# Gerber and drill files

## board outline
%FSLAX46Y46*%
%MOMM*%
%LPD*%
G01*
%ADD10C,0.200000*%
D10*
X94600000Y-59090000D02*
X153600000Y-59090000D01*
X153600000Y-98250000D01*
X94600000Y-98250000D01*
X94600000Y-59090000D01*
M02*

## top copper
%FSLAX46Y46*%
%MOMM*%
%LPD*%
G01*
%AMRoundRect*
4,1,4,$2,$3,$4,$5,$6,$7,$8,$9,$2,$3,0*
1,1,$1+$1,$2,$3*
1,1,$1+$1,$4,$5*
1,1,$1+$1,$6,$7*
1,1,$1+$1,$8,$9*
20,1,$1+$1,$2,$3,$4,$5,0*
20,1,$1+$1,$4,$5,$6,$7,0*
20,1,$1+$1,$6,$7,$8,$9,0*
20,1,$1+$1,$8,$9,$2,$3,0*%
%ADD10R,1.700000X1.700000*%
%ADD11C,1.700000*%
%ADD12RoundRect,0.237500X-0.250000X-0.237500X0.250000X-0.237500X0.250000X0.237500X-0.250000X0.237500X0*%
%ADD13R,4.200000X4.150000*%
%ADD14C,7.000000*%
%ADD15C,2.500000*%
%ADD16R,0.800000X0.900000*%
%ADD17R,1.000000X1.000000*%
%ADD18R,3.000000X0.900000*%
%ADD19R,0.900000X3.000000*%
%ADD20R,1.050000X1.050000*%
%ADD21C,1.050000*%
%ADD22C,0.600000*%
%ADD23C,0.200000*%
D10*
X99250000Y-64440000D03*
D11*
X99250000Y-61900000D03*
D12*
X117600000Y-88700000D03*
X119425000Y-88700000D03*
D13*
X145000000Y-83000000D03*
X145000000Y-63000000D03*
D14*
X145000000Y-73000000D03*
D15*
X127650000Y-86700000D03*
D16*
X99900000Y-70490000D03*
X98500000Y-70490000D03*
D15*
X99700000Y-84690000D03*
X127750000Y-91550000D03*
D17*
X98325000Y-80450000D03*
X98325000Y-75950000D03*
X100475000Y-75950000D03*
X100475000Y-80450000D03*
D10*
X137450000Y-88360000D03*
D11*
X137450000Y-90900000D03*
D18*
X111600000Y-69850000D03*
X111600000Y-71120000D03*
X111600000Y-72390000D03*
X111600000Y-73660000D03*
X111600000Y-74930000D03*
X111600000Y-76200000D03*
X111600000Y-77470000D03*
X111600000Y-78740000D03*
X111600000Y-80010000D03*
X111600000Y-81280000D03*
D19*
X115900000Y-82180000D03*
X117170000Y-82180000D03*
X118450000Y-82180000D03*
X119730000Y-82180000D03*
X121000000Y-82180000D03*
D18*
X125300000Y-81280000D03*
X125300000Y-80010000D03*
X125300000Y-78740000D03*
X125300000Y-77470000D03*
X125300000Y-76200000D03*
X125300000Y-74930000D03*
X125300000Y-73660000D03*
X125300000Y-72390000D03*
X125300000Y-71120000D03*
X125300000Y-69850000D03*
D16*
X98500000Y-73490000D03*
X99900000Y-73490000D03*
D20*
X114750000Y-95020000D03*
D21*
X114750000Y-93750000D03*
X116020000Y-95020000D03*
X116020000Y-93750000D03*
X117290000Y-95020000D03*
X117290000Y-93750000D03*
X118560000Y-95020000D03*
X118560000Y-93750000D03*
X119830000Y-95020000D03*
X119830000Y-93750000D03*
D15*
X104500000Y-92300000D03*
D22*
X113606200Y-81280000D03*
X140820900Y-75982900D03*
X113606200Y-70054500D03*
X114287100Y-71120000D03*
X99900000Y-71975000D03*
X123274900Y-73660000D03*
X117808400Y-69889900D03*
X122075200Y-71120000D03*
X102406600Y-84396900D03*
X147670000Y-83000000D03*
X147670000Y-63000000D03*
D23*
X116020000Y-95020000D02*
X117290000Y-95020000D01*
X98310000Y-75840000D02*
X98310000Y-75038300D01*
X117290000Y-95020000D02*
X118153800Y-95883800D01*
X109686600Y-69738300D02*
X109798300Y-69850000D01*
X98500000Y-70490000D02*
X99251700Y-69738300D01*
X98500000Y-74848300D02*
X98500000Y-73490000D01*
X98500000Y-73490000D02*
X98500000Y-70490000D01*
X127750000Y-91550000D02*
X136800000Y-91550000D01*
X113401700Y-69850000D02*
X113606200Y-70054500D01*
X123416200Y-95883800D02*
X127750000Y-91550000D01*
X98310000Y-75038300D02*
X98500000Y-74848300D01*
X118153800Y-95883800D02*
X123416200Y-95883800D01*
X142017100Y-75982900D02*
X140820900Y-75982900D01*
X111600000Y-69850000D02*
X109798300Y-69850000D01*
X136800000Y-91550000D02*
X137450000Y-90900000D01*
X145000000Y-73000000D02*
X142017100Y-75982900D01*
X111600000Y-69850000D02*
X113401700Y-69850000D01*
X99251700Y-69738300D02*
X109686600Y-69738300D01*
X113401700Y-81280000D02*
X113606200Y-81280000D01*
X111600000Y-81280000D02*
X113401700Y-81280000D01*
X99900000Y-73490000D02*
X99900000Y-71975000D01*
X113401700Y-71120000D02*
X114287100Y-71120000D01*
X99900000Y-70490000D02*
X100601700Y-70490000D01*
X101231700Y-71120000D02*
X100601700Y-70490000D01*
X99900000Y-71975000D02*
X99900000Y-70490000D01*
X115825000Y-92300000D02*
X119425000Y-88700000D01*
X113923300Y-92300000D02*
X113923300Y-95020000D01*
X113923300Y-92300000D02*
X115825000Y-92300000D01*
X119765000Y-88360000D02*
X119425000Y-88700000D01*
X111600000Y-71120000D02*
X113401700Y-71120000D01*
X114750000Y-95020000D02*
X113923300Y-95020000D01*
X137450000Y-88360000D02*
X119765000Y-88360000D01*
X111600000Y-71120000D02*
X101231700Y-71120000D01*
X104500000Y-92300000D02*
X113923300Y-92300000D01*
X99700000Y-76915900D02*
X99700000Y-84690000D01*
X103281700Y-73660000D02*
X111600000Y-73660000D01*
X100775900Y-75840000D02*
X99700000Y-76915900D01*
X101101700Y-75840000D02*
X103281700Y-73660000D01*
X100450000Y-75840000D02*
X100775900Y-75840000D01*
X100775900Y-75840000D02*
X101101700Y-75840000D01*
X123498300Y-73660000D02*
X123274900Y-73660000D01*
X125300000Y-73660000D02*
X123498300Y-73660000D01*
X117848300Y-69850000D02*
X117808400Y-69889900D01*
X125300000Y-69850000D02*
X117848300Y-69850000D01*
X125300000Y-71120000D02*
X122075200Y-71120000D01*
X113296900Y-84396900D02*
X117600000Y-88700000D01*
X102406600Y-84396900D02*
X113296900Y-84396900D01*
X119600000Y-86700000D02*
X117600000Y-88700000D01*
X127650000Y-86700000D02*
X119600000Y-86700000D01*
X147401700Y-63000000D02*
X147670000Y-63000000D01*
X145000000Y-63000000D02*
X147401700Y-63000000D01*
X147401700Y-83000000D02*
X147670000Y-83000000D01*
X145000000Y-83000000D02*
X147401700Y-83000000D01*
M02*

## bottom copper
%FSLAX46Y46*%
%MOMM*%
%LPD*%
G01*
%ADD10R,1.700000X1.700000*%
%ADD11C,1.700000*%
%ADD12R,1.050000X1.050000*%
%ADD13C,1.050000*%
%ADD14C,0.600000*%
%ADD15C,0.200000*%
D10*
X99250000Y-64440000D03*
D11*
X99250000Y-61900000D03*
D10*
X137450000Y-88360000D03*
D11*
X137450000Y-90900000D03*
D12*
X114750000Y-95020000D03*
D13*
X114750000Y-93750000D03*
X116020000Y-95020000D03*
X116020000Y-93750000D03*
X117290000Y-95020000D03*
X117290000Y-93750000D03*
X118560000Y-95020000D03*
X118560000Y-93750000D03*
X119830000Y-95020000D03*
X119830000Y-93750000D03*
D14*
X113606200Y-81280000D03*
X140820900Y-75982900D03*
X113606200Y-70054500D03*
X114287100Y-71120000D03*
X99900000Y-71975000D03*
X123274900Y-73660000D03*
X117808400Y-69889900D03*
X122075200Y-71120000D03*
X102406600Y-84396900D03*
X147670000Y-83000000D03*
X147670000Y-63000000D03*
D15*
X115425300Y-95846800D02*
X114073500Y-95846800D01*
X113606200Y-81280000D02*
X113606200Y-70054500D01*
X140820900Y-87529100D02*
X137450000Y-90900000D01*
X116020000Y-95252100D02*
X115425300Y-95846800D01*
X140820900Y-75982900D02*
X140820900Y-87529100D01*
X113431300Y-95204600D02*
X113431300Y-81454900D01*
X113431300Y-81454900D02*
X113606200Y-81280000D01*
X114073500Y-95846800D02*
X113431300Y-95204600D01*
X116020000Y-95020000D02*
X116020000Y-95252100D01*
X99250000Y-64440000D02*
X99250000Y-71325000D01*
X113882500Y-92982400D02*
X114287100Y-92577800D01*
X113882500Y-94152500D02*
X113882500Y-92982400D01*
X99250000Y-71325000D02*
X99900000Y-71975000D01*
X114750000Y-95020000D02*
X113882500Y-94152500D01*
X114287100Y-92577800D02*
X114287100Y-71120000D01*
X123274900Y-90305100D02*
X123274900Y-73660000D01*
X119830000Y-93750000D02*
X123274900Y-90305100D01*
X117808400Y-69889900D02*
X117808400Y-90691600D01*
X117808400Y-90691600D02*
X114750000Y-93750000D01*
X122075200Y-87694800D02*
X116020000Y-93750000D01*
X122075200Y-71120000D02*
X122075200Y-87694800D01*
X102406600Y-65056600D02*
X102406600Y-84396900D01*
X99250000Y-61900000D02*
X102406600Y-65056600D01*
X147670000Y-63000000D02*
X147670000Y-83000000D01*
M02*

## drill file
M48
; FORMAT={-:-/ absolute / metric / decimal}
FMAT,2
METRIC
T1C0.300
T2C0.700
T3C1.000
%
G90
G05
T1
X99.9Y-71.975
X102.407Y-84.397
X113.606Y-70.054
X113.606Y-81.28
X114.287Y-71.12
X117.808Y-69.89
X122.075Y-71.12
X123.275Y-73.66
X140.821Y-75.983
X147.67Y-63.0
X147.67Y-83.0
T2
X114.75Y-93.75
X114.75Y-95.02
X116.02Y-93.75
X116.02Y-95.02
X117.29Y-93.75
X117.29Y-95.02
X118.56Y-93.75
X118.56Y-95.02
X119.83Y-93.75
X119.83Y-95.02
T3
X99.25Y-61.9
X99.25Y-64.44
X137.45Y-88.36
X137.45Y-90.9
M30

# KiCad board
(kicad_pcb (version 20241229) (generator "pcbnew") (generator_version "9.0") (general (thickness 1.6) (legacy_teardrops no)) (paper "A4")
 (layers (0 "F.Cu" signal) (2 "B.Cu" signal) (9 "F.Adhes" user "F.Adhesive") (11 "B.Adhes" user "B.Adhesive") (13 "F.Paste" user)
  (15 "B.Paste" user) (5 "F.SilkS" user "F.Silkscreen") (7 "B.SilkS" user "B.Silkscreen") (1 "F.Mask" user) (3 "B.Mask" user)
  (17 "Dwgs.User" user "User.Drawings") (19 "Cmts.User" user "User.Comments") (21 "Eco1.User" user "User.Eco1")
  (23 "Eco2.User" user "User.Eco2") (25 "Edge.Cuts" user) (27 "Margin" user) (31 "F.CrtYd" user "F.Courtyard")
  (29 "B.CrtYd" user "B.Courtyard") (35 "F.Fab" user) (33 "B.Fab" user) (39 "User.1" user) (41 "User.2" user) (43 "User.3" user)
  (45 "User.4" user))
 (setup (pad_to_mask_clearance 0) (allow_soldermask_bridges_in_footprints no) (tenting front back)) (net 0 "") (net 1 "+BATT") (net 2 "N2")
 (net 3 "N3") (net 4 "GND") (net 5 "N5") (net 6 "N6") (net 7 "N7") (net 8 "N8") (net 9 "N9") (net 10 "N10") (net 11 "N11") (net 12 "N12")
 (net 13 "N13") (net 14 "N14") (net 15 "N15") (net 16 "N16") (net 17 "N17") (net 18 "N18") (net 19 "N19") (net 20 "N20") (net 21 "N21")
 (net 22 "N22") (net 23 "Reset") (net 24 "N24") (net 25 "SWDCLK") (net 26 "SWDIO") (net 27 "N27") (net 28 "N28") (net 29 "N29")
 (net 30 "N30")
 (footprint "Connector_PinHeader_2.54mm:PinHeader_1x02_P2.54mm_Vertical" (layer "F.Cu") (at 99.25 64.44 180)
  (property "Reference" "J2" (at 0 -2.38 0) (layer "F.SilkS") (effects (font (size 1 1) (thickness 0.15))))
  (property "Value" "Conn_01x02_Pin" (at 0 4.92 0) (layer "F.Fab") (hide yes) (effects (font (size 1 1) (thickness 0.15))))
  (pad "1" thru_hole rect (at 0 0 180) (size 1.7 1.7) (drill 1) (layers "*.Cu" "*.Mask") (remove_unused_layers no) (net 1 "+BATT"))
  (pad "2" thru_hole circle (at 0 2.54 180) (size 1.7 1.7) (drill 1) (layers "*.Cu" "*.Mask") (remove_unused_layers no) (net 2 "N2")))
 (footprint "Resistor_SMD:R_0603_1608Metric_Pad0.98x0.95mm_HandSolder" (layer "F.Cu") (at 118.5125 88.7)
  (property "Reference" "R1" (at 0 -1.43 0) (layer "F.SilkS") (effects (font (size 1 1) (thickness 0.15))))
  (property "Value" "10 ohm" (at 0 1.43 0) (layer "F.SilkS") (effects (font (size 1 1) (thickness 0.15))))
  (pad "1" smd roundrect (at -0.9125 0) (size 0.975 0.95) (layers "F.Cu" "F.Mask" "F.Paste") (roundrect_rratio 0.25) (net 2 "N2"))
  (pad "2" smd roundrect (at 0.9125 0) (size 0.975 0.95) (layers "F.Cu" "F.Mask" "F.Paste") (roundrect_rratio 0.25) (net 1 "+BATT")))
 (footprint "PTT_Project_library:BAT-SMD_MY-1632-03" (layer "F.Cu") (at 145 73 90)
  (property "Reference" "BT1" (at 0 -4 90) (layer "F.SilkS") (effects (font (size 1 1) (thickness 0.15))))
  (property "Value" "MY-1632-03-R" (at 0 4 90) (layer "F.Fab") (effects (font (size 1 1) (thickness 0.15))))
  (pad "1" smd rect (at -10 0 90) (size 4.15 4.2) (layers "F.Cu" "F.Mask" "F.Paste") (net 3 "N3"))
  (pad "1" smd rect (at 10 0 90) (size 4.15 4.2) (layers "F.Cu" "F.Mask" "F.Paste") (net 3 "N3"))
  (pad "2" smd circle (at 0 0 90) (size 7 7) (layers "F.Cu" "F.Mask" "F.Paste") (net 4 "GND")))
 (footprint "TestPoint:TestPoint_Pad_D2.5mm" (layer "F.Cu") (at 127.65 86.7 180)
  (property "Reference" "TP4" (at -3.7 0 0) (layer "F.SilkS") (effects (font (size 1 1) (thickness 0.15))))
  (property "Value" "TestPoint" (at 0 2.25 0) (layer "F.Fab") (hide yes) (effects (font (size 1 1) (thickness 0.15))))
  (pad "1" smd circle (at 0 0 180) (size 2.5 2.5) (layers "F.Cu" "F.Mask") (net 2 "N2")))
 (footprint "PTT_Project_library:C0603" (layer "F.Cu") (at 99.2 70.49 180)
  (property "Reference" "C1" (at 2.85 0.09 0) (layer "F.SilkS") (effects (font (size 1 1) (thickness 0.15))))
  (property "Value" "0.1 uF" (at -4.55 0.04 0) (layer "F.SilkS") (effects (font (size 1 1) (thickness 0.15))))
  (pad "1" smd rect (at -0.7 0 180) (size 0.8 0.9) (layers "F.Cu" "F.Mask" "F.Paste") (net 1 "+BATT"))
  (pad "2" smd rect (at 0.7 0 180) (size 0.8 0.9) (layers "F.Cu" "F.Mask" "F.Paste") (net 4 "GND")))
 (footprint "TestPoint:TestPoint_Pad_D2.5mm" (layer "F.Cu") (at 99.7 84.69)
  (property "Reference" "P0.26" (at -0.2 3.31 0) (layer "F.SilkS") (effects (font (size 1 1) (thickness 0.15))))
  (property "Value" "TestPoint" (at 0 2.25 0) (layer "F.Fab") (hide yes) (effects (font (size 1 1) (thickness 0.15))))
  (pad "1" smd circle (at 0 0) (size 2.5 2.5) (layers "F.Cu" "F.Mask") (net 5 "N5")))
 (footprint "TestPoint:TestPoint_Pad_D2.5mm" (layer "F.Cu") (at 127.75 91.55)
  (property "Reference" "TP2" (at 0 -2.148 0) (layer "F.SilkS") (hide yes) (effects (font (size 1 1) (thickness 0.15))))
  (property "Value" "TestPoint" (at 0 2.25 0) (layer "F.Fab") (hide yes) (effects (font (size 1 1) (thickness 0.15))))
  (pad "1" smd circle (at 0 0) (size 2.5 2.5) (layers "F.Cu" "F.Mask") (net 4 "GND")))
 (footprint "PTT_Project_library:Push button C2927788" (layer "F.Cu") (at 99.4 78.2 90)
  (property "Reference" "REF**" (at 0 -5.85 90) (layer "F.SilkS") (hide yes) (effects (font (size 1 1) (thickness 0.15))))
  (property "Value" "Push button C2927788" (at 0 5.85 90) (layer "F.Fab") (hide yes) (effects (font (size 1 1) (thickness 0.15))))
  (pad "1" smd rect (at -2.25 -1.075 90) (size 1 1) (layers "F.Cu" "F.Mask" "F.Paste"))
  (pad "2" smd rect (at 2.25 -1.075 90) (size 1 1) (layers "F.Cu" "F.Mask" "F.Paste"))
  (pad "3" smd rect (at 2.25 1.075 90) (size 1 1) (layers "F.Cu" "F.Mask" "F.Paste"))
  (pad "4" smd rect (at -2.25 1.075 90) (size 1 1) (layers "F.Cu" "F.Mask" "F.Paste")))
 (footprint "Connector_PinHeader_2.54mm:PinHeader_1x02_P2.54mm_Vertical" (layer "F.Cu") (at 137.45 88.36)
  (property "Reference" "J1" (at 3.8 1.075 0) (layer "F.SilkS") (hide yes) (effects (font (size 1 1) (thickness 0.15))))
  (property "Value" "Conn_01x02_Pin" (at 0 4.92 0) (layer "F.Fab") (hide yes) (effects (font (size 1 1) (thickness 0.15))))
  (pad "1" thru_hole rect (at 0 0) (size 1.7 1.7) (drill 1) (layers "*.Cu" "*.Mask") (remove_unused_layers no) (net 1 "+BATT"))
  (pad "2" thru_hole circle (at 0 2.54) (size 1.7 1.7) (drill 1) (layers "*.Cu" "*.Mask") (remove_unused_layers no) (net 4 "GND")))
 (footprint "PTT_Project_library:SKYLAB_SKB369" (layer "F.Cu") (at 118.45 73.48)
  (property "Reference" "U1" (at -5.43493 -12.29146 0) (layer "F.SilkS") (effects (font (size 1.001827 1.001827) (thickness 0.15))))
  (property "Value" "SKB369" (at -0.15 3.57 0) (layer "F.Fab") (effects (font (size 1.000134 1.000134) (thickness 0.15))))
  (pad "1" smd rect (at -6.85 -3.63) (size 3 0.9) (layers "F.Cu" "F.Mask" "F.Paste") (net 4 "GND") (solder_mask_margin 0.102))
  (pad "2" smd rect (at -6.85 -2.36) (size 3 0.9) (layers "F.Cu" "F.Mask" "F.Paste") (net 1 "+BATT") (solder_mask_margin 0.102))
  (pad "3" smd rect (at -6.85 -1.09) (size 3 0.9) (layers "F.Cu" "F.Mask" "F.Paste") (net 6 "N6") (solder_mask_margin 0.102))
  (pad "4" smd rect (at -6.85 0.18) (size 3 0.9) (layers "F.Cu" "F.Mask" "F.Paste") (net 5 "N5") (solder_mask_margin 0.102))
  (pad "5" smd rect (at -6.85 1.45) (size 3 0.9) (layers "F.Cu" "F.Mask" "F.Paste") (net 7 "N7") (solder_mask_margin 0.102))
  (pad "6" smd rect (at -6.85 2.72) (size 3 0.9) (layers "F.Cu" "F.Mask" "F.Paste") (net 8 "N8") (solder_mask_margin 0.102))
  (pad "7" smd rect (at -6.85 3.99) (size 3 0.9) (layers "F.Cu" "F.Mask" "F.Paste") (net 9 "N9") (solder_mask_margin 0.102))
  (pad "8" smd rect (at -6.85 5.26) (size 3 0.9) (layers "F.Cu" "F.Mask" "F.Paste") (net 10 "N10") (solder_mask_margin 0.102))
  (pad "9" smd rect (at -6.85 6.53) (size 3 0.9) (layers "F.Cu" "F.Mask" "F.Paste") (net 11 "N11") (solder_mask_margin 0.102))
  (pad "10" smd rect (at -6.85 7.8) (size 3 0.9) (layers "F.Cu" "F.Mask" "F.Paste") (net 4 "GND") (solder_mask_margin 0.102))
  (pad "11" smd rect (at -2.55 8.7) (size 0.9 3) (layers "F.Cu" "F.Mask" "F.Paste") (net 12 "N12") (solder_mask_margin 0.102))
  (pad "12" smd rect (at -1.28 8.7) (size 0.9 3) (layers "F.Cu" "F.Mask" "F.Paste") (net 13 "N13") (solder_mask_margin 0.102))
  (pad "13" smd rect (at 0 8.7) (size 0.9 3) (layers "F.Cu" "F.Mask" "F.Paste") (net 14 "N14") (solder_mask_margin 0.102))
  (pad "14" smd rect (at 1.28 8.7) (size 0.9 3) (layers "F.Cu" "F.Mask" "F.Paste") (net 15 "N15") (solder_mask_margin 0.102))
  (pad "15" smd rect (at 2.55 8.7) (size 0.9 3) (layers "F.Cu" "F.Mask" "F.Paste") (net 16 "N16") (solder_mask_margin 0.102))
  (pad "16" smd rect (at 6.85 7.8) (size 3 0.9) (layers "F.Cu" "F.Mask" "F.Paste") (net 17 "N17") (solder_mask_margin 0.102))
  (pad "17" smd rect (at 6.85 6.53) (size 3 0.9) (layers "F.Cu" "F.Mask" "F.Paste") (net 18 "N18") (solder_mask_margin 0.102))
  (pad "18" smd rect (at 6.85 5.26) (size 3 0.9) (layers "F.Cu" "F.Mask" "F.Paste") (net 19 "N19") (solder_mask_margin 0.102))
  (pad "19" smd rect (at 6.85 3.99) (size 3 0.9) (layers "F.Cu" "F.Mask" "F.Paste") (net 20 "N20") (solder_mask_margin 0.102))
  (pad "20" smd rect (at 6.85 2.72) (size 3 0.9) (layers "F.Cu" "F.Mask" "F.Paste") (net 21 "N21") (solder_mask_margin 0.102))
  (pad "21" smd rect (at 6.85 1.45) (size 3 0.9) (layers "F.Cu" "F.Mask" "F.Paste") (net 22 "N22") (solder_mask_margin 0.102))
  (pad "22" smd rect (at 6.85 0.18) (size 3 0.9) (layers "F.Cu" "F.Mask" "F.Paste") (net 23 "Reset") (solder_mask_margin 0.102))
  (pad "23" smd rect (at 6.85 -1.09) (size 3 0.9) (layers "F.Cu" "F.Mask" "F.Paste") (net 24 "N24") (solder_mask_margin 0.102))
  (pad "24" smd rect (at 6.85 -2.36) (size 3 0.9) (layers "F.Cu" "F.Mask" "F.Paste") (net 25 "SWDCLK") (solder_mask_margin 0.102))
  (pad "25" smd rect (at 6.85 -3.63) (size 3 0.9) (layers "F.Cu" "F.Mask" "F.Paste") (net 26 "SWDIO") (solder_mask_margin 0.102))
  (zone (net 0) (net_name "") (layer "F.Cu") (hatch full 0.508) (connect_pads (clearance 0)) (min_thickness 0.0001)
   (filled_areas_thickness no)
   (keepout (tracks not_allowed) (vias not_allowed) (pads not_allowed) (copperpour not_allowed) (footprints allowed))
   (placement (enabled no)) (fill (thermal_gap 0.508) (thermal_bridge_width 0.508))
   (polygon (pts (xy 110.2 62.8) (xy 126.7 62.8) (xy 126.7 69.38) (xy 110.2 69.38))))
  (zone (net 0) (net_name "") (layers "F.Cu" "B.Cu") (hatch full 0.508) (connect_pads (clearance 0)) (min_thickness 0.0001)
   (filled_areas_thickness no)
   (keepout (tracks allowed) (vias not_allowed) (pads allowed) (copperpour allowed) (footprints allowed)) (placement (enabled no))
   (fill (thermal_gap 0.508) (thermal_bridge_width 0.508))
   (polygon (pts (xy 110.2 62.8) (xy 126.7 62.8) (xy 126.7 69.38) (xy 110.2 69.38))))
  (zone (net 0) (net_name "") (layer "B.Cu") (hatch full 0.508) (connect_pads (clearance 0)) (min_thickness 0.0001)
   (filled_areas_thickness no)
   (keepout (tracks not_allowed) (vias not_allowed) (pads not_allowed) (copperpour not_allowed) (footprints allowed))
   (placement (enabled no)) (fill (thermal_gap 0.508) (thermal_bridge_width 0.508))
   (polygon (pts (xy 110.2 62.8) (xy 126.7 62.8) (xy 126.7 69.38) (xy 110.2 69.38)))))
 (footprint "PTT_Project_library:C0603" (layer "F.Cu") (at 99.2 73.49)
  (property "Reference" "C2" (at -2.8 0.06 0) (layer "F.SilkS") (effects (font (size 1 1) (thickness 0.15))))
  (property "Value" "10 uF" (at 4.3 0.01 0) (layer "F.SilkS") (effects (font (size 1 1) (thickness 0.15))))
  (pad "1" smd rect (at -0.7 0) (size 0.8 0.9) (layers "F.Cu" "F.Mask" "F.Paste") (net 4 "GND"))
  (pad "2" smd rect (at 0.7 0) (size 0.8 0.9) (layers "F.Cu" "F.Mask" "F.Paste") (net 1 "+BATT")))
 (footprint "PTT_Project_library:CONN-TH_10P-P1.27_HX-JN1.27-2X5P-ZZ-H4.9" (layer "F.Cu") (at 117.29 94.39)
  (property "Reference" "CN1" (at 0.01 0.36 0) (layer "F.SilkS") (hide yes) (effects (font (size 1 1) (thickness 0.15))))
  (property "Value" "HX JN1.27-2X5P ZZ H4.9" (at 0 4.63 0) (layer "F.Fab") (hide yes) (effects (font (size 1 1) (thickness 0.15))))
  (pad "1" thru_hole rect (at -2.54 0.63) (size 1.05 1.05) (drill 0.700024) (layers "*.Cu" "*.Mask") (remove_unused_layers no)
   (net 1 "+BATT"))
  (pad "2" thru_hole circle (at -2.54 -0.64) (size 1.05 1.05) (drill 0.700024) (layers "*.Cu" "*.Mask") (remove_unused_layers no)
   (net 26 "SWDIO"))
  (pad "3" thru_hole circle (at -1.27 0.63) (size 1.05 1.05) (drill 0.700024) (layers "*.Cu" "*.Mask") (remove_unused_layers no)
   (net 4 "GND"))
  (pad "4" thru_hole circle (at -1.27 -0.64) (size 1.05 1.05) (drill 0.700024) (layers "*.Cu" "*.Mask") (remove_unused_layers no)
   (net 25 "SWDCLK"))
  (pad "5" thru_hole circle (at 0 0.63) (size 1.05 1.05) (drill 0.700024) (layers "*.Cu" "*.Mask") (remove_unused_layers no) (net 4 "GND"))
  (pad "6" thru_hole circle (at 0 -0.64) (size 1.05 1.05) (drill 0.700024) (layers "*.Cu" "*.Mask") (remove_unused_layers no) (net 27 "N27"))
  (pad "7" thru_hole circle (at 1.27 0.63) (size 1.05 1.05) (drill 0.700024) (layers "*.Cu" "*.Mask") (remove_unused_layers no)
   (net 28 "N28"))
  (pad "8" thru_hole circle (at 1.27 -0.64) (size 1.05 1.05) (drill 0.700024) (layers "*.Cu" "*.Mask") (remove_unused_layers no)
   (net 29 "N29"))
  (pad "9" thru_hole circle (at 2.54 0.63) (size 1.05 1.05) (drill 0.700024) (layers "*.Cu" "*.Mask") (remove_unused_layers no)
   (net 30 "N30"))
  (pad "10" thru_hole circle (at 2.54 -0.64) (size 1.05 1.05) (drill 0.700024) (layers "*.Cu" "*.Mask") (remove_unused_layers no)
   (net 23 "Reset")))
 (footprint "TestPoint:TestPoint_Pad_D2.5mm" (layer "F.Cu") (at 104.5 92.3)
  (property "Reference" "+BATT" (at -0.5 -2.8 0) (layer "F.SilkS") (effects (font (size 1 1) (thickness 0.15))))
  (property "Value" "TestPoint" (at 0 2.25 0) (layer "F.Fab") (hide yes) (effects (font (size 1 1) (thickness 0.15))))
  (pad "1" smd circle (at 0 0) (size 2.5 2.5) (layers "F.Cu" "F.Mask") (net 1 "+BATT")))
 (gr_rect (start 94.6 59.09) (end 153.6 98.25) (stroke (width 0.2) (type solid)) (fill no) (layer "Edge.Cuts"))
 (segment (start 116.02 95.02) (end 117.29 95.02) (width 0.2) (layer "F.Cu") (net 4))
 (segment (start 98.31 75.84) (end 98.31 75.0383) (width 0.2) (layer "F.Cu") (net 4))
 (segment (start 117.29 95.02) (end 118.1538 95.8838) (width 0.2) (layer "F.Cu") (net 4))
 (segment (start 109.6866 69.7383) (end 109.7983 69.85) (width 0.2) (layer "F.Cu") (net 4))
 (segment (start 98.5 70.49) (end 99.2517 69.7383) (width 0.2) (layer "F.Cu") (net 4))
 (segment (start 98.5 74.8483) (end 98.5 73.49) (width 0.2) (layer "F.Cu") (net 4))
 (segment (start 98.5 73.49) (end 98.5 70.49) (width 0.2) (layer "F.Cu") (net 4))
 (segment (start 127.75 91.55) (end 136.8 91.55) (width 0.2) (layer "F.Cu") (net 4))
 (segment (start 113.4017 69.85) (end 113.6062 70.0545) (width 0.2) (layer "F.Cu") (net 4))
 (segment (start 123.4162 95.8838) (end 127.75 91.55) (width 0.2) (layer "F.Cu") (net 4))
 (segment (start 98.31 75.0383) (end 98.5 74.8483) (width 0.2) (layer "F.Cu") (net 4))
 (segment (start 118.1538 95.8838) (end 123.4162 95.8838) (width 0.2) (layer "F.Cu") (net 4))
 (segment (start 142.0171 75.9829) (end 140.8209 75.9829) (width 0.2) (layer "F.Cu") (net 4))
 (segment (start 111.6 69.85) (end 109.7983 69.85) (width 0.2) (layer "F.Cu") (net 4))
 (segment (start 136.8 91.55) (end 137.45 90.9) (width 0.2) (layer "F.Cu") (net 4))
 (segment (start 145 73) (end 142.0171 75.9829) (width 0.2) (layer "F.Cu") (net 4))
 (segment (start 111.6 69.85) (end 113.4017 69.85) (width 0.2) (layer "F.Cu") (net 4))
 (segment (start 99.2517 69.7383) (end 109.6866 69.7383) (width 0.2) (layer "F.Cu") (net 4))
 (segment (start 113.4017 81.28) (end 113.6062 81.28) (width 0.2) (layer "F.Cu") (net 4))
 (segment (start 111.6 81.28) (end 113.4017 81.28) (width 0.2) (layer "F.Cu") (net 4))
 (via (at 113.6062 81.28) (size 0.6) (drill 0.3) (layers "F.Cu" "B.Cu") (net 4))
 (via (at 140.8209 75.9829) (size 0.6) (drill 0.3) (layers "F.Cu" "B.Cu") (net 4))
 (via (at 113.6062 70.0545) (size 0.6) (drill 0.3) (layers "F.Cu" "B.Cu") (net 4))
 (segment (start 115.4253 95.8468) (end 114.0735 95.8468) (width 0.2) (layer "B.Cu") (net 4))
 (segment (start 113.6062 81.28) (end 113.6062 70.0545) (width 0.2) (layer "B.Cu") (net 4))
 (segment (start 140.8209 87.5291) (end 137.45 90.9) (width 0.2) (layer "B.Cu") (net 4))
 (segment (start 116.02 95.2521) (end 115.4253 95.8468) (width 0.2) (layer "B.Cu") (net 4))
 (segment (start 140.8209 75.9829) (end 140.8209 87.5291) (width 0.2) (layer "B.Cu") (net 4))
 (segment (start 113.4313 95.2046) (end 113.4313 81.4549) (width 0.2) (layer "B.Cu") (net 4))
 (segment (start 113.4313 81.4549) (end 113.6062 81.28) (width 0.2) (layer "B.Cu") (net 4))
 (segment (start 114.0735 95.8468) (end 113.4313 95.2046) (width 0.2) (layer "B.Cu") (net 4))
 (segment (start 116.02 95.02) (end 116.02 95.2521) (width 0.2) (layer "B.Cu") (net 4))
 (segment (start 99.9 73.49) (end 99.9 71.975) (width 0.2) (layer "F.Cu") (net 1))
 (segment (start 113.4017 71.12) (end 114.2871 71.12) (width 0.2) (layer "F.Cu") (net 1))
 (segment (start 99.9 70.49) (end 100.6017 70.49) (width 0.2) (layer "F.Cu") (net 1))
 (segment (start 101.2317 71.12) (end 100.6017 70.49) (width 0.2) (layer "F.Cu") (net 1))
 (segment (start 99.9 71.975) (end 99.9 70.49) (width 0.2) (layer "F.Cu") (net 1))
 (segment (start 115.825 92.3) (end 119.425 88.7) (width 0.2) (layer "F.Cu") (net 1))
 (segment (start 113.9233 92.3) (end 113.9233 95.02) (width 0.2) (layer "F.Cu") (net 1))
 (segment (start 113.9233 92.3) (end 115.825 92.3) (width 0.2) (layer "F.Cu") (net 1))
 (segment (start 119.765 88.36) (end 119.425 88.7) (width 0.2) (layer "F.Cu") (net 1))
 (segment (start 111.6 71.12) (end 113.4017 71.12) (width 0.2) (layer "F.Cu") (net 1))
 (segment (start 114.75 95.02) (end 113.9233 95.02) (width 0.2) (layer "F.Cu") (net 1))
 (segment (start 137.45 88.36) (end 119.765 88.36) (width 0.2) (layer "F.Cu") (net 1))
 (segment (start 111.6 71.12) (end 101.2317 71.12) (width 0.2) (layer "F.Cu") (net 1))
 (segment (start 104.5 92.3) (end 113.9233 92.3) (width 0.2) (layer "F.Cu") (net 1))
 (via (at 114.2871 71.12) (size 0.6) (drill 0.3) (layers "F.Cu" "B.Cu") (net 1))
 (via (at 99.9 71.975) (size 0.6) (drill 0.3) (layers "F.Cu" "B.Cu") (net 1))
 (segment (start 99.25 64.44) (end 99.25 71.325) (width 0.2) (layer "B.Cu") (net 1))
 (segment (start 113.8825 92.9824) (end 114.2871 92.5778) (width 0.2) (layer "B.Cu") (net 1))
 (segment (start 113.8825 94.1525) (end 113.8825 92.9824) (width 0.2) (layer "B.Cu") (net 1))
 (segment (start 99.25 71.325) (end 99.9 71.975) (width 0.2) (layer "B.Cu") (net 1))
 (segment (start 114.75 95.02) (end 113.8825 94.1525) (width 0.2) (layer "B.Cu") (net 1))
 (segment (start 114.2871 92.5778) (end 114.2871 71.12) (width 0.2) (layer "B.Cu") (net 1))
 (segment (start 99.7 76.9159) (end 99.7 84.69) (width 0.2) (layer "F.Cu") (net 5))
 (segment (start 103.2817 73.66) (end 111.6 73.66) (width 0.2) (layer "F.Cu") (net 5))
 (segment (start 100.7759 75.84) (end 99.7 76.9159) (width 0.2) (layer "F.Cu") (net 5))
 (segment (start 101.1017 75.84) (end 103.2817 73.66) (width 0.2) (layer "F.Cu") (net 5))
 (segment (start 100.45 75.84) (end 100.7759 75.84) (width 0.2) (layer "F.Cu") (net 5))
 (segment (start 100.7759 75.84) (end 101.1017 75.84) (width 0.2) (layer "F.Cu") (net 5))
 (segment (start 123.4983 73.66) (end 123.2749 73.66) (width 0.2) (layer "F.Cu") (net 23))
 (segment (start 125.3 73.66) (end 123.4983 73.66) (width 0.2) (layer "F.Cu") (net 23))
 (via (at 123.2749 73.66) (size 0.6) (drill 0.3) (layers "F.Cu" "B.Cu") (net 23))
 (segment (start 123.2749 90.3051) (end 123.2749 73.66) (width 0.2) (layer "B.Cu") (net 23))
 (segment (start 119.83 93.75) (end 123.2749 90.3051) (width 0.2) (layer "B.Cu") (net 23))
 (segment (start 117.8483 69.85) (end 117.8084 69.8899) (width 0.2) (layer "F.Cu") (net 26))
 (segment (start 125.3 69.85) (end 117.8483 69.85) (width 0.2) (layer "F.Cu") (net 26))
 (via (at 117.8084 69.8899) (size 0.6) (drill 0.3) (layers "F.Cu" "B.Cu") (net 26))
 (segment (start 117.8084 69.8899) (end 117.8084 90.6916) (width 0.2) (layer "B.Cu") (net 26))
 (segment (start 117.8084 90.6916) (end 114.75 93.75) (width 0.2) (layer "B.Cu") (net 26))
 (segment (start 125.3 71.12) (end 122.0752 71.12) (width 0.2) (layer "F.Cu") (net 25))
 (via (at 122.0752 71.12) (size 0.6) (drill 0.3) (layers "F.Cu" "B.Cu") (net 25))
 (segment (start 122.0752 87.6948) (end 116.02 93.75) (width 0.2) (layer "B.Cu") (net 25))
 (segment (start 122.0752 71.12) (end 122.0752 87.6948) (width 0.2) (layer "B.Cu") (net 25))
 (segment (start 113.2969 84.3969) (end 117.6 88.7) (width 0.2) (layer "F.Cu") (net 2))
 (segment (start 102.4066 84.3969) (end 113.2969 84.3969) (width 0.2) (layer "F.Cu") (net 2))
 (segment (start 119.6 86.7) (end 117.6 88.7) (width 0.2) (layer "F.Cu") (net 2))
 (segment (start 127.65 86.7) (end 119.6 86.7) (width 0.2) (layer "F.Cu") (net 2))
 (via (at 102.4066 84.3969) (size 0.6) (drill 0.3) (layers "F.Cu" "B.Cu") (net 2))
 (segment (start 102.4066 65.0566) (end 102.4066 84.3969) (width 0.2) (layer "B.Cu") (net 2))
 (segment (start 99.25 61.9) (end 102.4066 65.0566) (width 0.2) (layer "B.Cu") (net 2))
 (segment (start 147.4017 63) (end 147.67 63) (width 0.2) (layer "F.Cu") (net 3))
 (segment (start 145 63) (end 147.4017 63) (width 0.2) (layer "F.Cu") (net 3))
 (segment (start 147.4017 83) (end 147.67 83) (width 0.2) (layer "F.Cu") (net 3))
 (segment (start 145 83) (end 147.4017 83) (width 0.2) (layer "F.Cu") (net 3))
 (via (at 147.67 83) (size 0.6) (drill 0.3) (layers "F.Cu" "B.Cu") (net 3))
 (via (at 147.67 63) (size 0.6) (drill 0.3) (layers "F.Cu" "B.Cu") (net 3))
 (segment (start 147.67 63) (end 147.67 83) (width 0.2) (layer "B.Cu") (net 3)))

